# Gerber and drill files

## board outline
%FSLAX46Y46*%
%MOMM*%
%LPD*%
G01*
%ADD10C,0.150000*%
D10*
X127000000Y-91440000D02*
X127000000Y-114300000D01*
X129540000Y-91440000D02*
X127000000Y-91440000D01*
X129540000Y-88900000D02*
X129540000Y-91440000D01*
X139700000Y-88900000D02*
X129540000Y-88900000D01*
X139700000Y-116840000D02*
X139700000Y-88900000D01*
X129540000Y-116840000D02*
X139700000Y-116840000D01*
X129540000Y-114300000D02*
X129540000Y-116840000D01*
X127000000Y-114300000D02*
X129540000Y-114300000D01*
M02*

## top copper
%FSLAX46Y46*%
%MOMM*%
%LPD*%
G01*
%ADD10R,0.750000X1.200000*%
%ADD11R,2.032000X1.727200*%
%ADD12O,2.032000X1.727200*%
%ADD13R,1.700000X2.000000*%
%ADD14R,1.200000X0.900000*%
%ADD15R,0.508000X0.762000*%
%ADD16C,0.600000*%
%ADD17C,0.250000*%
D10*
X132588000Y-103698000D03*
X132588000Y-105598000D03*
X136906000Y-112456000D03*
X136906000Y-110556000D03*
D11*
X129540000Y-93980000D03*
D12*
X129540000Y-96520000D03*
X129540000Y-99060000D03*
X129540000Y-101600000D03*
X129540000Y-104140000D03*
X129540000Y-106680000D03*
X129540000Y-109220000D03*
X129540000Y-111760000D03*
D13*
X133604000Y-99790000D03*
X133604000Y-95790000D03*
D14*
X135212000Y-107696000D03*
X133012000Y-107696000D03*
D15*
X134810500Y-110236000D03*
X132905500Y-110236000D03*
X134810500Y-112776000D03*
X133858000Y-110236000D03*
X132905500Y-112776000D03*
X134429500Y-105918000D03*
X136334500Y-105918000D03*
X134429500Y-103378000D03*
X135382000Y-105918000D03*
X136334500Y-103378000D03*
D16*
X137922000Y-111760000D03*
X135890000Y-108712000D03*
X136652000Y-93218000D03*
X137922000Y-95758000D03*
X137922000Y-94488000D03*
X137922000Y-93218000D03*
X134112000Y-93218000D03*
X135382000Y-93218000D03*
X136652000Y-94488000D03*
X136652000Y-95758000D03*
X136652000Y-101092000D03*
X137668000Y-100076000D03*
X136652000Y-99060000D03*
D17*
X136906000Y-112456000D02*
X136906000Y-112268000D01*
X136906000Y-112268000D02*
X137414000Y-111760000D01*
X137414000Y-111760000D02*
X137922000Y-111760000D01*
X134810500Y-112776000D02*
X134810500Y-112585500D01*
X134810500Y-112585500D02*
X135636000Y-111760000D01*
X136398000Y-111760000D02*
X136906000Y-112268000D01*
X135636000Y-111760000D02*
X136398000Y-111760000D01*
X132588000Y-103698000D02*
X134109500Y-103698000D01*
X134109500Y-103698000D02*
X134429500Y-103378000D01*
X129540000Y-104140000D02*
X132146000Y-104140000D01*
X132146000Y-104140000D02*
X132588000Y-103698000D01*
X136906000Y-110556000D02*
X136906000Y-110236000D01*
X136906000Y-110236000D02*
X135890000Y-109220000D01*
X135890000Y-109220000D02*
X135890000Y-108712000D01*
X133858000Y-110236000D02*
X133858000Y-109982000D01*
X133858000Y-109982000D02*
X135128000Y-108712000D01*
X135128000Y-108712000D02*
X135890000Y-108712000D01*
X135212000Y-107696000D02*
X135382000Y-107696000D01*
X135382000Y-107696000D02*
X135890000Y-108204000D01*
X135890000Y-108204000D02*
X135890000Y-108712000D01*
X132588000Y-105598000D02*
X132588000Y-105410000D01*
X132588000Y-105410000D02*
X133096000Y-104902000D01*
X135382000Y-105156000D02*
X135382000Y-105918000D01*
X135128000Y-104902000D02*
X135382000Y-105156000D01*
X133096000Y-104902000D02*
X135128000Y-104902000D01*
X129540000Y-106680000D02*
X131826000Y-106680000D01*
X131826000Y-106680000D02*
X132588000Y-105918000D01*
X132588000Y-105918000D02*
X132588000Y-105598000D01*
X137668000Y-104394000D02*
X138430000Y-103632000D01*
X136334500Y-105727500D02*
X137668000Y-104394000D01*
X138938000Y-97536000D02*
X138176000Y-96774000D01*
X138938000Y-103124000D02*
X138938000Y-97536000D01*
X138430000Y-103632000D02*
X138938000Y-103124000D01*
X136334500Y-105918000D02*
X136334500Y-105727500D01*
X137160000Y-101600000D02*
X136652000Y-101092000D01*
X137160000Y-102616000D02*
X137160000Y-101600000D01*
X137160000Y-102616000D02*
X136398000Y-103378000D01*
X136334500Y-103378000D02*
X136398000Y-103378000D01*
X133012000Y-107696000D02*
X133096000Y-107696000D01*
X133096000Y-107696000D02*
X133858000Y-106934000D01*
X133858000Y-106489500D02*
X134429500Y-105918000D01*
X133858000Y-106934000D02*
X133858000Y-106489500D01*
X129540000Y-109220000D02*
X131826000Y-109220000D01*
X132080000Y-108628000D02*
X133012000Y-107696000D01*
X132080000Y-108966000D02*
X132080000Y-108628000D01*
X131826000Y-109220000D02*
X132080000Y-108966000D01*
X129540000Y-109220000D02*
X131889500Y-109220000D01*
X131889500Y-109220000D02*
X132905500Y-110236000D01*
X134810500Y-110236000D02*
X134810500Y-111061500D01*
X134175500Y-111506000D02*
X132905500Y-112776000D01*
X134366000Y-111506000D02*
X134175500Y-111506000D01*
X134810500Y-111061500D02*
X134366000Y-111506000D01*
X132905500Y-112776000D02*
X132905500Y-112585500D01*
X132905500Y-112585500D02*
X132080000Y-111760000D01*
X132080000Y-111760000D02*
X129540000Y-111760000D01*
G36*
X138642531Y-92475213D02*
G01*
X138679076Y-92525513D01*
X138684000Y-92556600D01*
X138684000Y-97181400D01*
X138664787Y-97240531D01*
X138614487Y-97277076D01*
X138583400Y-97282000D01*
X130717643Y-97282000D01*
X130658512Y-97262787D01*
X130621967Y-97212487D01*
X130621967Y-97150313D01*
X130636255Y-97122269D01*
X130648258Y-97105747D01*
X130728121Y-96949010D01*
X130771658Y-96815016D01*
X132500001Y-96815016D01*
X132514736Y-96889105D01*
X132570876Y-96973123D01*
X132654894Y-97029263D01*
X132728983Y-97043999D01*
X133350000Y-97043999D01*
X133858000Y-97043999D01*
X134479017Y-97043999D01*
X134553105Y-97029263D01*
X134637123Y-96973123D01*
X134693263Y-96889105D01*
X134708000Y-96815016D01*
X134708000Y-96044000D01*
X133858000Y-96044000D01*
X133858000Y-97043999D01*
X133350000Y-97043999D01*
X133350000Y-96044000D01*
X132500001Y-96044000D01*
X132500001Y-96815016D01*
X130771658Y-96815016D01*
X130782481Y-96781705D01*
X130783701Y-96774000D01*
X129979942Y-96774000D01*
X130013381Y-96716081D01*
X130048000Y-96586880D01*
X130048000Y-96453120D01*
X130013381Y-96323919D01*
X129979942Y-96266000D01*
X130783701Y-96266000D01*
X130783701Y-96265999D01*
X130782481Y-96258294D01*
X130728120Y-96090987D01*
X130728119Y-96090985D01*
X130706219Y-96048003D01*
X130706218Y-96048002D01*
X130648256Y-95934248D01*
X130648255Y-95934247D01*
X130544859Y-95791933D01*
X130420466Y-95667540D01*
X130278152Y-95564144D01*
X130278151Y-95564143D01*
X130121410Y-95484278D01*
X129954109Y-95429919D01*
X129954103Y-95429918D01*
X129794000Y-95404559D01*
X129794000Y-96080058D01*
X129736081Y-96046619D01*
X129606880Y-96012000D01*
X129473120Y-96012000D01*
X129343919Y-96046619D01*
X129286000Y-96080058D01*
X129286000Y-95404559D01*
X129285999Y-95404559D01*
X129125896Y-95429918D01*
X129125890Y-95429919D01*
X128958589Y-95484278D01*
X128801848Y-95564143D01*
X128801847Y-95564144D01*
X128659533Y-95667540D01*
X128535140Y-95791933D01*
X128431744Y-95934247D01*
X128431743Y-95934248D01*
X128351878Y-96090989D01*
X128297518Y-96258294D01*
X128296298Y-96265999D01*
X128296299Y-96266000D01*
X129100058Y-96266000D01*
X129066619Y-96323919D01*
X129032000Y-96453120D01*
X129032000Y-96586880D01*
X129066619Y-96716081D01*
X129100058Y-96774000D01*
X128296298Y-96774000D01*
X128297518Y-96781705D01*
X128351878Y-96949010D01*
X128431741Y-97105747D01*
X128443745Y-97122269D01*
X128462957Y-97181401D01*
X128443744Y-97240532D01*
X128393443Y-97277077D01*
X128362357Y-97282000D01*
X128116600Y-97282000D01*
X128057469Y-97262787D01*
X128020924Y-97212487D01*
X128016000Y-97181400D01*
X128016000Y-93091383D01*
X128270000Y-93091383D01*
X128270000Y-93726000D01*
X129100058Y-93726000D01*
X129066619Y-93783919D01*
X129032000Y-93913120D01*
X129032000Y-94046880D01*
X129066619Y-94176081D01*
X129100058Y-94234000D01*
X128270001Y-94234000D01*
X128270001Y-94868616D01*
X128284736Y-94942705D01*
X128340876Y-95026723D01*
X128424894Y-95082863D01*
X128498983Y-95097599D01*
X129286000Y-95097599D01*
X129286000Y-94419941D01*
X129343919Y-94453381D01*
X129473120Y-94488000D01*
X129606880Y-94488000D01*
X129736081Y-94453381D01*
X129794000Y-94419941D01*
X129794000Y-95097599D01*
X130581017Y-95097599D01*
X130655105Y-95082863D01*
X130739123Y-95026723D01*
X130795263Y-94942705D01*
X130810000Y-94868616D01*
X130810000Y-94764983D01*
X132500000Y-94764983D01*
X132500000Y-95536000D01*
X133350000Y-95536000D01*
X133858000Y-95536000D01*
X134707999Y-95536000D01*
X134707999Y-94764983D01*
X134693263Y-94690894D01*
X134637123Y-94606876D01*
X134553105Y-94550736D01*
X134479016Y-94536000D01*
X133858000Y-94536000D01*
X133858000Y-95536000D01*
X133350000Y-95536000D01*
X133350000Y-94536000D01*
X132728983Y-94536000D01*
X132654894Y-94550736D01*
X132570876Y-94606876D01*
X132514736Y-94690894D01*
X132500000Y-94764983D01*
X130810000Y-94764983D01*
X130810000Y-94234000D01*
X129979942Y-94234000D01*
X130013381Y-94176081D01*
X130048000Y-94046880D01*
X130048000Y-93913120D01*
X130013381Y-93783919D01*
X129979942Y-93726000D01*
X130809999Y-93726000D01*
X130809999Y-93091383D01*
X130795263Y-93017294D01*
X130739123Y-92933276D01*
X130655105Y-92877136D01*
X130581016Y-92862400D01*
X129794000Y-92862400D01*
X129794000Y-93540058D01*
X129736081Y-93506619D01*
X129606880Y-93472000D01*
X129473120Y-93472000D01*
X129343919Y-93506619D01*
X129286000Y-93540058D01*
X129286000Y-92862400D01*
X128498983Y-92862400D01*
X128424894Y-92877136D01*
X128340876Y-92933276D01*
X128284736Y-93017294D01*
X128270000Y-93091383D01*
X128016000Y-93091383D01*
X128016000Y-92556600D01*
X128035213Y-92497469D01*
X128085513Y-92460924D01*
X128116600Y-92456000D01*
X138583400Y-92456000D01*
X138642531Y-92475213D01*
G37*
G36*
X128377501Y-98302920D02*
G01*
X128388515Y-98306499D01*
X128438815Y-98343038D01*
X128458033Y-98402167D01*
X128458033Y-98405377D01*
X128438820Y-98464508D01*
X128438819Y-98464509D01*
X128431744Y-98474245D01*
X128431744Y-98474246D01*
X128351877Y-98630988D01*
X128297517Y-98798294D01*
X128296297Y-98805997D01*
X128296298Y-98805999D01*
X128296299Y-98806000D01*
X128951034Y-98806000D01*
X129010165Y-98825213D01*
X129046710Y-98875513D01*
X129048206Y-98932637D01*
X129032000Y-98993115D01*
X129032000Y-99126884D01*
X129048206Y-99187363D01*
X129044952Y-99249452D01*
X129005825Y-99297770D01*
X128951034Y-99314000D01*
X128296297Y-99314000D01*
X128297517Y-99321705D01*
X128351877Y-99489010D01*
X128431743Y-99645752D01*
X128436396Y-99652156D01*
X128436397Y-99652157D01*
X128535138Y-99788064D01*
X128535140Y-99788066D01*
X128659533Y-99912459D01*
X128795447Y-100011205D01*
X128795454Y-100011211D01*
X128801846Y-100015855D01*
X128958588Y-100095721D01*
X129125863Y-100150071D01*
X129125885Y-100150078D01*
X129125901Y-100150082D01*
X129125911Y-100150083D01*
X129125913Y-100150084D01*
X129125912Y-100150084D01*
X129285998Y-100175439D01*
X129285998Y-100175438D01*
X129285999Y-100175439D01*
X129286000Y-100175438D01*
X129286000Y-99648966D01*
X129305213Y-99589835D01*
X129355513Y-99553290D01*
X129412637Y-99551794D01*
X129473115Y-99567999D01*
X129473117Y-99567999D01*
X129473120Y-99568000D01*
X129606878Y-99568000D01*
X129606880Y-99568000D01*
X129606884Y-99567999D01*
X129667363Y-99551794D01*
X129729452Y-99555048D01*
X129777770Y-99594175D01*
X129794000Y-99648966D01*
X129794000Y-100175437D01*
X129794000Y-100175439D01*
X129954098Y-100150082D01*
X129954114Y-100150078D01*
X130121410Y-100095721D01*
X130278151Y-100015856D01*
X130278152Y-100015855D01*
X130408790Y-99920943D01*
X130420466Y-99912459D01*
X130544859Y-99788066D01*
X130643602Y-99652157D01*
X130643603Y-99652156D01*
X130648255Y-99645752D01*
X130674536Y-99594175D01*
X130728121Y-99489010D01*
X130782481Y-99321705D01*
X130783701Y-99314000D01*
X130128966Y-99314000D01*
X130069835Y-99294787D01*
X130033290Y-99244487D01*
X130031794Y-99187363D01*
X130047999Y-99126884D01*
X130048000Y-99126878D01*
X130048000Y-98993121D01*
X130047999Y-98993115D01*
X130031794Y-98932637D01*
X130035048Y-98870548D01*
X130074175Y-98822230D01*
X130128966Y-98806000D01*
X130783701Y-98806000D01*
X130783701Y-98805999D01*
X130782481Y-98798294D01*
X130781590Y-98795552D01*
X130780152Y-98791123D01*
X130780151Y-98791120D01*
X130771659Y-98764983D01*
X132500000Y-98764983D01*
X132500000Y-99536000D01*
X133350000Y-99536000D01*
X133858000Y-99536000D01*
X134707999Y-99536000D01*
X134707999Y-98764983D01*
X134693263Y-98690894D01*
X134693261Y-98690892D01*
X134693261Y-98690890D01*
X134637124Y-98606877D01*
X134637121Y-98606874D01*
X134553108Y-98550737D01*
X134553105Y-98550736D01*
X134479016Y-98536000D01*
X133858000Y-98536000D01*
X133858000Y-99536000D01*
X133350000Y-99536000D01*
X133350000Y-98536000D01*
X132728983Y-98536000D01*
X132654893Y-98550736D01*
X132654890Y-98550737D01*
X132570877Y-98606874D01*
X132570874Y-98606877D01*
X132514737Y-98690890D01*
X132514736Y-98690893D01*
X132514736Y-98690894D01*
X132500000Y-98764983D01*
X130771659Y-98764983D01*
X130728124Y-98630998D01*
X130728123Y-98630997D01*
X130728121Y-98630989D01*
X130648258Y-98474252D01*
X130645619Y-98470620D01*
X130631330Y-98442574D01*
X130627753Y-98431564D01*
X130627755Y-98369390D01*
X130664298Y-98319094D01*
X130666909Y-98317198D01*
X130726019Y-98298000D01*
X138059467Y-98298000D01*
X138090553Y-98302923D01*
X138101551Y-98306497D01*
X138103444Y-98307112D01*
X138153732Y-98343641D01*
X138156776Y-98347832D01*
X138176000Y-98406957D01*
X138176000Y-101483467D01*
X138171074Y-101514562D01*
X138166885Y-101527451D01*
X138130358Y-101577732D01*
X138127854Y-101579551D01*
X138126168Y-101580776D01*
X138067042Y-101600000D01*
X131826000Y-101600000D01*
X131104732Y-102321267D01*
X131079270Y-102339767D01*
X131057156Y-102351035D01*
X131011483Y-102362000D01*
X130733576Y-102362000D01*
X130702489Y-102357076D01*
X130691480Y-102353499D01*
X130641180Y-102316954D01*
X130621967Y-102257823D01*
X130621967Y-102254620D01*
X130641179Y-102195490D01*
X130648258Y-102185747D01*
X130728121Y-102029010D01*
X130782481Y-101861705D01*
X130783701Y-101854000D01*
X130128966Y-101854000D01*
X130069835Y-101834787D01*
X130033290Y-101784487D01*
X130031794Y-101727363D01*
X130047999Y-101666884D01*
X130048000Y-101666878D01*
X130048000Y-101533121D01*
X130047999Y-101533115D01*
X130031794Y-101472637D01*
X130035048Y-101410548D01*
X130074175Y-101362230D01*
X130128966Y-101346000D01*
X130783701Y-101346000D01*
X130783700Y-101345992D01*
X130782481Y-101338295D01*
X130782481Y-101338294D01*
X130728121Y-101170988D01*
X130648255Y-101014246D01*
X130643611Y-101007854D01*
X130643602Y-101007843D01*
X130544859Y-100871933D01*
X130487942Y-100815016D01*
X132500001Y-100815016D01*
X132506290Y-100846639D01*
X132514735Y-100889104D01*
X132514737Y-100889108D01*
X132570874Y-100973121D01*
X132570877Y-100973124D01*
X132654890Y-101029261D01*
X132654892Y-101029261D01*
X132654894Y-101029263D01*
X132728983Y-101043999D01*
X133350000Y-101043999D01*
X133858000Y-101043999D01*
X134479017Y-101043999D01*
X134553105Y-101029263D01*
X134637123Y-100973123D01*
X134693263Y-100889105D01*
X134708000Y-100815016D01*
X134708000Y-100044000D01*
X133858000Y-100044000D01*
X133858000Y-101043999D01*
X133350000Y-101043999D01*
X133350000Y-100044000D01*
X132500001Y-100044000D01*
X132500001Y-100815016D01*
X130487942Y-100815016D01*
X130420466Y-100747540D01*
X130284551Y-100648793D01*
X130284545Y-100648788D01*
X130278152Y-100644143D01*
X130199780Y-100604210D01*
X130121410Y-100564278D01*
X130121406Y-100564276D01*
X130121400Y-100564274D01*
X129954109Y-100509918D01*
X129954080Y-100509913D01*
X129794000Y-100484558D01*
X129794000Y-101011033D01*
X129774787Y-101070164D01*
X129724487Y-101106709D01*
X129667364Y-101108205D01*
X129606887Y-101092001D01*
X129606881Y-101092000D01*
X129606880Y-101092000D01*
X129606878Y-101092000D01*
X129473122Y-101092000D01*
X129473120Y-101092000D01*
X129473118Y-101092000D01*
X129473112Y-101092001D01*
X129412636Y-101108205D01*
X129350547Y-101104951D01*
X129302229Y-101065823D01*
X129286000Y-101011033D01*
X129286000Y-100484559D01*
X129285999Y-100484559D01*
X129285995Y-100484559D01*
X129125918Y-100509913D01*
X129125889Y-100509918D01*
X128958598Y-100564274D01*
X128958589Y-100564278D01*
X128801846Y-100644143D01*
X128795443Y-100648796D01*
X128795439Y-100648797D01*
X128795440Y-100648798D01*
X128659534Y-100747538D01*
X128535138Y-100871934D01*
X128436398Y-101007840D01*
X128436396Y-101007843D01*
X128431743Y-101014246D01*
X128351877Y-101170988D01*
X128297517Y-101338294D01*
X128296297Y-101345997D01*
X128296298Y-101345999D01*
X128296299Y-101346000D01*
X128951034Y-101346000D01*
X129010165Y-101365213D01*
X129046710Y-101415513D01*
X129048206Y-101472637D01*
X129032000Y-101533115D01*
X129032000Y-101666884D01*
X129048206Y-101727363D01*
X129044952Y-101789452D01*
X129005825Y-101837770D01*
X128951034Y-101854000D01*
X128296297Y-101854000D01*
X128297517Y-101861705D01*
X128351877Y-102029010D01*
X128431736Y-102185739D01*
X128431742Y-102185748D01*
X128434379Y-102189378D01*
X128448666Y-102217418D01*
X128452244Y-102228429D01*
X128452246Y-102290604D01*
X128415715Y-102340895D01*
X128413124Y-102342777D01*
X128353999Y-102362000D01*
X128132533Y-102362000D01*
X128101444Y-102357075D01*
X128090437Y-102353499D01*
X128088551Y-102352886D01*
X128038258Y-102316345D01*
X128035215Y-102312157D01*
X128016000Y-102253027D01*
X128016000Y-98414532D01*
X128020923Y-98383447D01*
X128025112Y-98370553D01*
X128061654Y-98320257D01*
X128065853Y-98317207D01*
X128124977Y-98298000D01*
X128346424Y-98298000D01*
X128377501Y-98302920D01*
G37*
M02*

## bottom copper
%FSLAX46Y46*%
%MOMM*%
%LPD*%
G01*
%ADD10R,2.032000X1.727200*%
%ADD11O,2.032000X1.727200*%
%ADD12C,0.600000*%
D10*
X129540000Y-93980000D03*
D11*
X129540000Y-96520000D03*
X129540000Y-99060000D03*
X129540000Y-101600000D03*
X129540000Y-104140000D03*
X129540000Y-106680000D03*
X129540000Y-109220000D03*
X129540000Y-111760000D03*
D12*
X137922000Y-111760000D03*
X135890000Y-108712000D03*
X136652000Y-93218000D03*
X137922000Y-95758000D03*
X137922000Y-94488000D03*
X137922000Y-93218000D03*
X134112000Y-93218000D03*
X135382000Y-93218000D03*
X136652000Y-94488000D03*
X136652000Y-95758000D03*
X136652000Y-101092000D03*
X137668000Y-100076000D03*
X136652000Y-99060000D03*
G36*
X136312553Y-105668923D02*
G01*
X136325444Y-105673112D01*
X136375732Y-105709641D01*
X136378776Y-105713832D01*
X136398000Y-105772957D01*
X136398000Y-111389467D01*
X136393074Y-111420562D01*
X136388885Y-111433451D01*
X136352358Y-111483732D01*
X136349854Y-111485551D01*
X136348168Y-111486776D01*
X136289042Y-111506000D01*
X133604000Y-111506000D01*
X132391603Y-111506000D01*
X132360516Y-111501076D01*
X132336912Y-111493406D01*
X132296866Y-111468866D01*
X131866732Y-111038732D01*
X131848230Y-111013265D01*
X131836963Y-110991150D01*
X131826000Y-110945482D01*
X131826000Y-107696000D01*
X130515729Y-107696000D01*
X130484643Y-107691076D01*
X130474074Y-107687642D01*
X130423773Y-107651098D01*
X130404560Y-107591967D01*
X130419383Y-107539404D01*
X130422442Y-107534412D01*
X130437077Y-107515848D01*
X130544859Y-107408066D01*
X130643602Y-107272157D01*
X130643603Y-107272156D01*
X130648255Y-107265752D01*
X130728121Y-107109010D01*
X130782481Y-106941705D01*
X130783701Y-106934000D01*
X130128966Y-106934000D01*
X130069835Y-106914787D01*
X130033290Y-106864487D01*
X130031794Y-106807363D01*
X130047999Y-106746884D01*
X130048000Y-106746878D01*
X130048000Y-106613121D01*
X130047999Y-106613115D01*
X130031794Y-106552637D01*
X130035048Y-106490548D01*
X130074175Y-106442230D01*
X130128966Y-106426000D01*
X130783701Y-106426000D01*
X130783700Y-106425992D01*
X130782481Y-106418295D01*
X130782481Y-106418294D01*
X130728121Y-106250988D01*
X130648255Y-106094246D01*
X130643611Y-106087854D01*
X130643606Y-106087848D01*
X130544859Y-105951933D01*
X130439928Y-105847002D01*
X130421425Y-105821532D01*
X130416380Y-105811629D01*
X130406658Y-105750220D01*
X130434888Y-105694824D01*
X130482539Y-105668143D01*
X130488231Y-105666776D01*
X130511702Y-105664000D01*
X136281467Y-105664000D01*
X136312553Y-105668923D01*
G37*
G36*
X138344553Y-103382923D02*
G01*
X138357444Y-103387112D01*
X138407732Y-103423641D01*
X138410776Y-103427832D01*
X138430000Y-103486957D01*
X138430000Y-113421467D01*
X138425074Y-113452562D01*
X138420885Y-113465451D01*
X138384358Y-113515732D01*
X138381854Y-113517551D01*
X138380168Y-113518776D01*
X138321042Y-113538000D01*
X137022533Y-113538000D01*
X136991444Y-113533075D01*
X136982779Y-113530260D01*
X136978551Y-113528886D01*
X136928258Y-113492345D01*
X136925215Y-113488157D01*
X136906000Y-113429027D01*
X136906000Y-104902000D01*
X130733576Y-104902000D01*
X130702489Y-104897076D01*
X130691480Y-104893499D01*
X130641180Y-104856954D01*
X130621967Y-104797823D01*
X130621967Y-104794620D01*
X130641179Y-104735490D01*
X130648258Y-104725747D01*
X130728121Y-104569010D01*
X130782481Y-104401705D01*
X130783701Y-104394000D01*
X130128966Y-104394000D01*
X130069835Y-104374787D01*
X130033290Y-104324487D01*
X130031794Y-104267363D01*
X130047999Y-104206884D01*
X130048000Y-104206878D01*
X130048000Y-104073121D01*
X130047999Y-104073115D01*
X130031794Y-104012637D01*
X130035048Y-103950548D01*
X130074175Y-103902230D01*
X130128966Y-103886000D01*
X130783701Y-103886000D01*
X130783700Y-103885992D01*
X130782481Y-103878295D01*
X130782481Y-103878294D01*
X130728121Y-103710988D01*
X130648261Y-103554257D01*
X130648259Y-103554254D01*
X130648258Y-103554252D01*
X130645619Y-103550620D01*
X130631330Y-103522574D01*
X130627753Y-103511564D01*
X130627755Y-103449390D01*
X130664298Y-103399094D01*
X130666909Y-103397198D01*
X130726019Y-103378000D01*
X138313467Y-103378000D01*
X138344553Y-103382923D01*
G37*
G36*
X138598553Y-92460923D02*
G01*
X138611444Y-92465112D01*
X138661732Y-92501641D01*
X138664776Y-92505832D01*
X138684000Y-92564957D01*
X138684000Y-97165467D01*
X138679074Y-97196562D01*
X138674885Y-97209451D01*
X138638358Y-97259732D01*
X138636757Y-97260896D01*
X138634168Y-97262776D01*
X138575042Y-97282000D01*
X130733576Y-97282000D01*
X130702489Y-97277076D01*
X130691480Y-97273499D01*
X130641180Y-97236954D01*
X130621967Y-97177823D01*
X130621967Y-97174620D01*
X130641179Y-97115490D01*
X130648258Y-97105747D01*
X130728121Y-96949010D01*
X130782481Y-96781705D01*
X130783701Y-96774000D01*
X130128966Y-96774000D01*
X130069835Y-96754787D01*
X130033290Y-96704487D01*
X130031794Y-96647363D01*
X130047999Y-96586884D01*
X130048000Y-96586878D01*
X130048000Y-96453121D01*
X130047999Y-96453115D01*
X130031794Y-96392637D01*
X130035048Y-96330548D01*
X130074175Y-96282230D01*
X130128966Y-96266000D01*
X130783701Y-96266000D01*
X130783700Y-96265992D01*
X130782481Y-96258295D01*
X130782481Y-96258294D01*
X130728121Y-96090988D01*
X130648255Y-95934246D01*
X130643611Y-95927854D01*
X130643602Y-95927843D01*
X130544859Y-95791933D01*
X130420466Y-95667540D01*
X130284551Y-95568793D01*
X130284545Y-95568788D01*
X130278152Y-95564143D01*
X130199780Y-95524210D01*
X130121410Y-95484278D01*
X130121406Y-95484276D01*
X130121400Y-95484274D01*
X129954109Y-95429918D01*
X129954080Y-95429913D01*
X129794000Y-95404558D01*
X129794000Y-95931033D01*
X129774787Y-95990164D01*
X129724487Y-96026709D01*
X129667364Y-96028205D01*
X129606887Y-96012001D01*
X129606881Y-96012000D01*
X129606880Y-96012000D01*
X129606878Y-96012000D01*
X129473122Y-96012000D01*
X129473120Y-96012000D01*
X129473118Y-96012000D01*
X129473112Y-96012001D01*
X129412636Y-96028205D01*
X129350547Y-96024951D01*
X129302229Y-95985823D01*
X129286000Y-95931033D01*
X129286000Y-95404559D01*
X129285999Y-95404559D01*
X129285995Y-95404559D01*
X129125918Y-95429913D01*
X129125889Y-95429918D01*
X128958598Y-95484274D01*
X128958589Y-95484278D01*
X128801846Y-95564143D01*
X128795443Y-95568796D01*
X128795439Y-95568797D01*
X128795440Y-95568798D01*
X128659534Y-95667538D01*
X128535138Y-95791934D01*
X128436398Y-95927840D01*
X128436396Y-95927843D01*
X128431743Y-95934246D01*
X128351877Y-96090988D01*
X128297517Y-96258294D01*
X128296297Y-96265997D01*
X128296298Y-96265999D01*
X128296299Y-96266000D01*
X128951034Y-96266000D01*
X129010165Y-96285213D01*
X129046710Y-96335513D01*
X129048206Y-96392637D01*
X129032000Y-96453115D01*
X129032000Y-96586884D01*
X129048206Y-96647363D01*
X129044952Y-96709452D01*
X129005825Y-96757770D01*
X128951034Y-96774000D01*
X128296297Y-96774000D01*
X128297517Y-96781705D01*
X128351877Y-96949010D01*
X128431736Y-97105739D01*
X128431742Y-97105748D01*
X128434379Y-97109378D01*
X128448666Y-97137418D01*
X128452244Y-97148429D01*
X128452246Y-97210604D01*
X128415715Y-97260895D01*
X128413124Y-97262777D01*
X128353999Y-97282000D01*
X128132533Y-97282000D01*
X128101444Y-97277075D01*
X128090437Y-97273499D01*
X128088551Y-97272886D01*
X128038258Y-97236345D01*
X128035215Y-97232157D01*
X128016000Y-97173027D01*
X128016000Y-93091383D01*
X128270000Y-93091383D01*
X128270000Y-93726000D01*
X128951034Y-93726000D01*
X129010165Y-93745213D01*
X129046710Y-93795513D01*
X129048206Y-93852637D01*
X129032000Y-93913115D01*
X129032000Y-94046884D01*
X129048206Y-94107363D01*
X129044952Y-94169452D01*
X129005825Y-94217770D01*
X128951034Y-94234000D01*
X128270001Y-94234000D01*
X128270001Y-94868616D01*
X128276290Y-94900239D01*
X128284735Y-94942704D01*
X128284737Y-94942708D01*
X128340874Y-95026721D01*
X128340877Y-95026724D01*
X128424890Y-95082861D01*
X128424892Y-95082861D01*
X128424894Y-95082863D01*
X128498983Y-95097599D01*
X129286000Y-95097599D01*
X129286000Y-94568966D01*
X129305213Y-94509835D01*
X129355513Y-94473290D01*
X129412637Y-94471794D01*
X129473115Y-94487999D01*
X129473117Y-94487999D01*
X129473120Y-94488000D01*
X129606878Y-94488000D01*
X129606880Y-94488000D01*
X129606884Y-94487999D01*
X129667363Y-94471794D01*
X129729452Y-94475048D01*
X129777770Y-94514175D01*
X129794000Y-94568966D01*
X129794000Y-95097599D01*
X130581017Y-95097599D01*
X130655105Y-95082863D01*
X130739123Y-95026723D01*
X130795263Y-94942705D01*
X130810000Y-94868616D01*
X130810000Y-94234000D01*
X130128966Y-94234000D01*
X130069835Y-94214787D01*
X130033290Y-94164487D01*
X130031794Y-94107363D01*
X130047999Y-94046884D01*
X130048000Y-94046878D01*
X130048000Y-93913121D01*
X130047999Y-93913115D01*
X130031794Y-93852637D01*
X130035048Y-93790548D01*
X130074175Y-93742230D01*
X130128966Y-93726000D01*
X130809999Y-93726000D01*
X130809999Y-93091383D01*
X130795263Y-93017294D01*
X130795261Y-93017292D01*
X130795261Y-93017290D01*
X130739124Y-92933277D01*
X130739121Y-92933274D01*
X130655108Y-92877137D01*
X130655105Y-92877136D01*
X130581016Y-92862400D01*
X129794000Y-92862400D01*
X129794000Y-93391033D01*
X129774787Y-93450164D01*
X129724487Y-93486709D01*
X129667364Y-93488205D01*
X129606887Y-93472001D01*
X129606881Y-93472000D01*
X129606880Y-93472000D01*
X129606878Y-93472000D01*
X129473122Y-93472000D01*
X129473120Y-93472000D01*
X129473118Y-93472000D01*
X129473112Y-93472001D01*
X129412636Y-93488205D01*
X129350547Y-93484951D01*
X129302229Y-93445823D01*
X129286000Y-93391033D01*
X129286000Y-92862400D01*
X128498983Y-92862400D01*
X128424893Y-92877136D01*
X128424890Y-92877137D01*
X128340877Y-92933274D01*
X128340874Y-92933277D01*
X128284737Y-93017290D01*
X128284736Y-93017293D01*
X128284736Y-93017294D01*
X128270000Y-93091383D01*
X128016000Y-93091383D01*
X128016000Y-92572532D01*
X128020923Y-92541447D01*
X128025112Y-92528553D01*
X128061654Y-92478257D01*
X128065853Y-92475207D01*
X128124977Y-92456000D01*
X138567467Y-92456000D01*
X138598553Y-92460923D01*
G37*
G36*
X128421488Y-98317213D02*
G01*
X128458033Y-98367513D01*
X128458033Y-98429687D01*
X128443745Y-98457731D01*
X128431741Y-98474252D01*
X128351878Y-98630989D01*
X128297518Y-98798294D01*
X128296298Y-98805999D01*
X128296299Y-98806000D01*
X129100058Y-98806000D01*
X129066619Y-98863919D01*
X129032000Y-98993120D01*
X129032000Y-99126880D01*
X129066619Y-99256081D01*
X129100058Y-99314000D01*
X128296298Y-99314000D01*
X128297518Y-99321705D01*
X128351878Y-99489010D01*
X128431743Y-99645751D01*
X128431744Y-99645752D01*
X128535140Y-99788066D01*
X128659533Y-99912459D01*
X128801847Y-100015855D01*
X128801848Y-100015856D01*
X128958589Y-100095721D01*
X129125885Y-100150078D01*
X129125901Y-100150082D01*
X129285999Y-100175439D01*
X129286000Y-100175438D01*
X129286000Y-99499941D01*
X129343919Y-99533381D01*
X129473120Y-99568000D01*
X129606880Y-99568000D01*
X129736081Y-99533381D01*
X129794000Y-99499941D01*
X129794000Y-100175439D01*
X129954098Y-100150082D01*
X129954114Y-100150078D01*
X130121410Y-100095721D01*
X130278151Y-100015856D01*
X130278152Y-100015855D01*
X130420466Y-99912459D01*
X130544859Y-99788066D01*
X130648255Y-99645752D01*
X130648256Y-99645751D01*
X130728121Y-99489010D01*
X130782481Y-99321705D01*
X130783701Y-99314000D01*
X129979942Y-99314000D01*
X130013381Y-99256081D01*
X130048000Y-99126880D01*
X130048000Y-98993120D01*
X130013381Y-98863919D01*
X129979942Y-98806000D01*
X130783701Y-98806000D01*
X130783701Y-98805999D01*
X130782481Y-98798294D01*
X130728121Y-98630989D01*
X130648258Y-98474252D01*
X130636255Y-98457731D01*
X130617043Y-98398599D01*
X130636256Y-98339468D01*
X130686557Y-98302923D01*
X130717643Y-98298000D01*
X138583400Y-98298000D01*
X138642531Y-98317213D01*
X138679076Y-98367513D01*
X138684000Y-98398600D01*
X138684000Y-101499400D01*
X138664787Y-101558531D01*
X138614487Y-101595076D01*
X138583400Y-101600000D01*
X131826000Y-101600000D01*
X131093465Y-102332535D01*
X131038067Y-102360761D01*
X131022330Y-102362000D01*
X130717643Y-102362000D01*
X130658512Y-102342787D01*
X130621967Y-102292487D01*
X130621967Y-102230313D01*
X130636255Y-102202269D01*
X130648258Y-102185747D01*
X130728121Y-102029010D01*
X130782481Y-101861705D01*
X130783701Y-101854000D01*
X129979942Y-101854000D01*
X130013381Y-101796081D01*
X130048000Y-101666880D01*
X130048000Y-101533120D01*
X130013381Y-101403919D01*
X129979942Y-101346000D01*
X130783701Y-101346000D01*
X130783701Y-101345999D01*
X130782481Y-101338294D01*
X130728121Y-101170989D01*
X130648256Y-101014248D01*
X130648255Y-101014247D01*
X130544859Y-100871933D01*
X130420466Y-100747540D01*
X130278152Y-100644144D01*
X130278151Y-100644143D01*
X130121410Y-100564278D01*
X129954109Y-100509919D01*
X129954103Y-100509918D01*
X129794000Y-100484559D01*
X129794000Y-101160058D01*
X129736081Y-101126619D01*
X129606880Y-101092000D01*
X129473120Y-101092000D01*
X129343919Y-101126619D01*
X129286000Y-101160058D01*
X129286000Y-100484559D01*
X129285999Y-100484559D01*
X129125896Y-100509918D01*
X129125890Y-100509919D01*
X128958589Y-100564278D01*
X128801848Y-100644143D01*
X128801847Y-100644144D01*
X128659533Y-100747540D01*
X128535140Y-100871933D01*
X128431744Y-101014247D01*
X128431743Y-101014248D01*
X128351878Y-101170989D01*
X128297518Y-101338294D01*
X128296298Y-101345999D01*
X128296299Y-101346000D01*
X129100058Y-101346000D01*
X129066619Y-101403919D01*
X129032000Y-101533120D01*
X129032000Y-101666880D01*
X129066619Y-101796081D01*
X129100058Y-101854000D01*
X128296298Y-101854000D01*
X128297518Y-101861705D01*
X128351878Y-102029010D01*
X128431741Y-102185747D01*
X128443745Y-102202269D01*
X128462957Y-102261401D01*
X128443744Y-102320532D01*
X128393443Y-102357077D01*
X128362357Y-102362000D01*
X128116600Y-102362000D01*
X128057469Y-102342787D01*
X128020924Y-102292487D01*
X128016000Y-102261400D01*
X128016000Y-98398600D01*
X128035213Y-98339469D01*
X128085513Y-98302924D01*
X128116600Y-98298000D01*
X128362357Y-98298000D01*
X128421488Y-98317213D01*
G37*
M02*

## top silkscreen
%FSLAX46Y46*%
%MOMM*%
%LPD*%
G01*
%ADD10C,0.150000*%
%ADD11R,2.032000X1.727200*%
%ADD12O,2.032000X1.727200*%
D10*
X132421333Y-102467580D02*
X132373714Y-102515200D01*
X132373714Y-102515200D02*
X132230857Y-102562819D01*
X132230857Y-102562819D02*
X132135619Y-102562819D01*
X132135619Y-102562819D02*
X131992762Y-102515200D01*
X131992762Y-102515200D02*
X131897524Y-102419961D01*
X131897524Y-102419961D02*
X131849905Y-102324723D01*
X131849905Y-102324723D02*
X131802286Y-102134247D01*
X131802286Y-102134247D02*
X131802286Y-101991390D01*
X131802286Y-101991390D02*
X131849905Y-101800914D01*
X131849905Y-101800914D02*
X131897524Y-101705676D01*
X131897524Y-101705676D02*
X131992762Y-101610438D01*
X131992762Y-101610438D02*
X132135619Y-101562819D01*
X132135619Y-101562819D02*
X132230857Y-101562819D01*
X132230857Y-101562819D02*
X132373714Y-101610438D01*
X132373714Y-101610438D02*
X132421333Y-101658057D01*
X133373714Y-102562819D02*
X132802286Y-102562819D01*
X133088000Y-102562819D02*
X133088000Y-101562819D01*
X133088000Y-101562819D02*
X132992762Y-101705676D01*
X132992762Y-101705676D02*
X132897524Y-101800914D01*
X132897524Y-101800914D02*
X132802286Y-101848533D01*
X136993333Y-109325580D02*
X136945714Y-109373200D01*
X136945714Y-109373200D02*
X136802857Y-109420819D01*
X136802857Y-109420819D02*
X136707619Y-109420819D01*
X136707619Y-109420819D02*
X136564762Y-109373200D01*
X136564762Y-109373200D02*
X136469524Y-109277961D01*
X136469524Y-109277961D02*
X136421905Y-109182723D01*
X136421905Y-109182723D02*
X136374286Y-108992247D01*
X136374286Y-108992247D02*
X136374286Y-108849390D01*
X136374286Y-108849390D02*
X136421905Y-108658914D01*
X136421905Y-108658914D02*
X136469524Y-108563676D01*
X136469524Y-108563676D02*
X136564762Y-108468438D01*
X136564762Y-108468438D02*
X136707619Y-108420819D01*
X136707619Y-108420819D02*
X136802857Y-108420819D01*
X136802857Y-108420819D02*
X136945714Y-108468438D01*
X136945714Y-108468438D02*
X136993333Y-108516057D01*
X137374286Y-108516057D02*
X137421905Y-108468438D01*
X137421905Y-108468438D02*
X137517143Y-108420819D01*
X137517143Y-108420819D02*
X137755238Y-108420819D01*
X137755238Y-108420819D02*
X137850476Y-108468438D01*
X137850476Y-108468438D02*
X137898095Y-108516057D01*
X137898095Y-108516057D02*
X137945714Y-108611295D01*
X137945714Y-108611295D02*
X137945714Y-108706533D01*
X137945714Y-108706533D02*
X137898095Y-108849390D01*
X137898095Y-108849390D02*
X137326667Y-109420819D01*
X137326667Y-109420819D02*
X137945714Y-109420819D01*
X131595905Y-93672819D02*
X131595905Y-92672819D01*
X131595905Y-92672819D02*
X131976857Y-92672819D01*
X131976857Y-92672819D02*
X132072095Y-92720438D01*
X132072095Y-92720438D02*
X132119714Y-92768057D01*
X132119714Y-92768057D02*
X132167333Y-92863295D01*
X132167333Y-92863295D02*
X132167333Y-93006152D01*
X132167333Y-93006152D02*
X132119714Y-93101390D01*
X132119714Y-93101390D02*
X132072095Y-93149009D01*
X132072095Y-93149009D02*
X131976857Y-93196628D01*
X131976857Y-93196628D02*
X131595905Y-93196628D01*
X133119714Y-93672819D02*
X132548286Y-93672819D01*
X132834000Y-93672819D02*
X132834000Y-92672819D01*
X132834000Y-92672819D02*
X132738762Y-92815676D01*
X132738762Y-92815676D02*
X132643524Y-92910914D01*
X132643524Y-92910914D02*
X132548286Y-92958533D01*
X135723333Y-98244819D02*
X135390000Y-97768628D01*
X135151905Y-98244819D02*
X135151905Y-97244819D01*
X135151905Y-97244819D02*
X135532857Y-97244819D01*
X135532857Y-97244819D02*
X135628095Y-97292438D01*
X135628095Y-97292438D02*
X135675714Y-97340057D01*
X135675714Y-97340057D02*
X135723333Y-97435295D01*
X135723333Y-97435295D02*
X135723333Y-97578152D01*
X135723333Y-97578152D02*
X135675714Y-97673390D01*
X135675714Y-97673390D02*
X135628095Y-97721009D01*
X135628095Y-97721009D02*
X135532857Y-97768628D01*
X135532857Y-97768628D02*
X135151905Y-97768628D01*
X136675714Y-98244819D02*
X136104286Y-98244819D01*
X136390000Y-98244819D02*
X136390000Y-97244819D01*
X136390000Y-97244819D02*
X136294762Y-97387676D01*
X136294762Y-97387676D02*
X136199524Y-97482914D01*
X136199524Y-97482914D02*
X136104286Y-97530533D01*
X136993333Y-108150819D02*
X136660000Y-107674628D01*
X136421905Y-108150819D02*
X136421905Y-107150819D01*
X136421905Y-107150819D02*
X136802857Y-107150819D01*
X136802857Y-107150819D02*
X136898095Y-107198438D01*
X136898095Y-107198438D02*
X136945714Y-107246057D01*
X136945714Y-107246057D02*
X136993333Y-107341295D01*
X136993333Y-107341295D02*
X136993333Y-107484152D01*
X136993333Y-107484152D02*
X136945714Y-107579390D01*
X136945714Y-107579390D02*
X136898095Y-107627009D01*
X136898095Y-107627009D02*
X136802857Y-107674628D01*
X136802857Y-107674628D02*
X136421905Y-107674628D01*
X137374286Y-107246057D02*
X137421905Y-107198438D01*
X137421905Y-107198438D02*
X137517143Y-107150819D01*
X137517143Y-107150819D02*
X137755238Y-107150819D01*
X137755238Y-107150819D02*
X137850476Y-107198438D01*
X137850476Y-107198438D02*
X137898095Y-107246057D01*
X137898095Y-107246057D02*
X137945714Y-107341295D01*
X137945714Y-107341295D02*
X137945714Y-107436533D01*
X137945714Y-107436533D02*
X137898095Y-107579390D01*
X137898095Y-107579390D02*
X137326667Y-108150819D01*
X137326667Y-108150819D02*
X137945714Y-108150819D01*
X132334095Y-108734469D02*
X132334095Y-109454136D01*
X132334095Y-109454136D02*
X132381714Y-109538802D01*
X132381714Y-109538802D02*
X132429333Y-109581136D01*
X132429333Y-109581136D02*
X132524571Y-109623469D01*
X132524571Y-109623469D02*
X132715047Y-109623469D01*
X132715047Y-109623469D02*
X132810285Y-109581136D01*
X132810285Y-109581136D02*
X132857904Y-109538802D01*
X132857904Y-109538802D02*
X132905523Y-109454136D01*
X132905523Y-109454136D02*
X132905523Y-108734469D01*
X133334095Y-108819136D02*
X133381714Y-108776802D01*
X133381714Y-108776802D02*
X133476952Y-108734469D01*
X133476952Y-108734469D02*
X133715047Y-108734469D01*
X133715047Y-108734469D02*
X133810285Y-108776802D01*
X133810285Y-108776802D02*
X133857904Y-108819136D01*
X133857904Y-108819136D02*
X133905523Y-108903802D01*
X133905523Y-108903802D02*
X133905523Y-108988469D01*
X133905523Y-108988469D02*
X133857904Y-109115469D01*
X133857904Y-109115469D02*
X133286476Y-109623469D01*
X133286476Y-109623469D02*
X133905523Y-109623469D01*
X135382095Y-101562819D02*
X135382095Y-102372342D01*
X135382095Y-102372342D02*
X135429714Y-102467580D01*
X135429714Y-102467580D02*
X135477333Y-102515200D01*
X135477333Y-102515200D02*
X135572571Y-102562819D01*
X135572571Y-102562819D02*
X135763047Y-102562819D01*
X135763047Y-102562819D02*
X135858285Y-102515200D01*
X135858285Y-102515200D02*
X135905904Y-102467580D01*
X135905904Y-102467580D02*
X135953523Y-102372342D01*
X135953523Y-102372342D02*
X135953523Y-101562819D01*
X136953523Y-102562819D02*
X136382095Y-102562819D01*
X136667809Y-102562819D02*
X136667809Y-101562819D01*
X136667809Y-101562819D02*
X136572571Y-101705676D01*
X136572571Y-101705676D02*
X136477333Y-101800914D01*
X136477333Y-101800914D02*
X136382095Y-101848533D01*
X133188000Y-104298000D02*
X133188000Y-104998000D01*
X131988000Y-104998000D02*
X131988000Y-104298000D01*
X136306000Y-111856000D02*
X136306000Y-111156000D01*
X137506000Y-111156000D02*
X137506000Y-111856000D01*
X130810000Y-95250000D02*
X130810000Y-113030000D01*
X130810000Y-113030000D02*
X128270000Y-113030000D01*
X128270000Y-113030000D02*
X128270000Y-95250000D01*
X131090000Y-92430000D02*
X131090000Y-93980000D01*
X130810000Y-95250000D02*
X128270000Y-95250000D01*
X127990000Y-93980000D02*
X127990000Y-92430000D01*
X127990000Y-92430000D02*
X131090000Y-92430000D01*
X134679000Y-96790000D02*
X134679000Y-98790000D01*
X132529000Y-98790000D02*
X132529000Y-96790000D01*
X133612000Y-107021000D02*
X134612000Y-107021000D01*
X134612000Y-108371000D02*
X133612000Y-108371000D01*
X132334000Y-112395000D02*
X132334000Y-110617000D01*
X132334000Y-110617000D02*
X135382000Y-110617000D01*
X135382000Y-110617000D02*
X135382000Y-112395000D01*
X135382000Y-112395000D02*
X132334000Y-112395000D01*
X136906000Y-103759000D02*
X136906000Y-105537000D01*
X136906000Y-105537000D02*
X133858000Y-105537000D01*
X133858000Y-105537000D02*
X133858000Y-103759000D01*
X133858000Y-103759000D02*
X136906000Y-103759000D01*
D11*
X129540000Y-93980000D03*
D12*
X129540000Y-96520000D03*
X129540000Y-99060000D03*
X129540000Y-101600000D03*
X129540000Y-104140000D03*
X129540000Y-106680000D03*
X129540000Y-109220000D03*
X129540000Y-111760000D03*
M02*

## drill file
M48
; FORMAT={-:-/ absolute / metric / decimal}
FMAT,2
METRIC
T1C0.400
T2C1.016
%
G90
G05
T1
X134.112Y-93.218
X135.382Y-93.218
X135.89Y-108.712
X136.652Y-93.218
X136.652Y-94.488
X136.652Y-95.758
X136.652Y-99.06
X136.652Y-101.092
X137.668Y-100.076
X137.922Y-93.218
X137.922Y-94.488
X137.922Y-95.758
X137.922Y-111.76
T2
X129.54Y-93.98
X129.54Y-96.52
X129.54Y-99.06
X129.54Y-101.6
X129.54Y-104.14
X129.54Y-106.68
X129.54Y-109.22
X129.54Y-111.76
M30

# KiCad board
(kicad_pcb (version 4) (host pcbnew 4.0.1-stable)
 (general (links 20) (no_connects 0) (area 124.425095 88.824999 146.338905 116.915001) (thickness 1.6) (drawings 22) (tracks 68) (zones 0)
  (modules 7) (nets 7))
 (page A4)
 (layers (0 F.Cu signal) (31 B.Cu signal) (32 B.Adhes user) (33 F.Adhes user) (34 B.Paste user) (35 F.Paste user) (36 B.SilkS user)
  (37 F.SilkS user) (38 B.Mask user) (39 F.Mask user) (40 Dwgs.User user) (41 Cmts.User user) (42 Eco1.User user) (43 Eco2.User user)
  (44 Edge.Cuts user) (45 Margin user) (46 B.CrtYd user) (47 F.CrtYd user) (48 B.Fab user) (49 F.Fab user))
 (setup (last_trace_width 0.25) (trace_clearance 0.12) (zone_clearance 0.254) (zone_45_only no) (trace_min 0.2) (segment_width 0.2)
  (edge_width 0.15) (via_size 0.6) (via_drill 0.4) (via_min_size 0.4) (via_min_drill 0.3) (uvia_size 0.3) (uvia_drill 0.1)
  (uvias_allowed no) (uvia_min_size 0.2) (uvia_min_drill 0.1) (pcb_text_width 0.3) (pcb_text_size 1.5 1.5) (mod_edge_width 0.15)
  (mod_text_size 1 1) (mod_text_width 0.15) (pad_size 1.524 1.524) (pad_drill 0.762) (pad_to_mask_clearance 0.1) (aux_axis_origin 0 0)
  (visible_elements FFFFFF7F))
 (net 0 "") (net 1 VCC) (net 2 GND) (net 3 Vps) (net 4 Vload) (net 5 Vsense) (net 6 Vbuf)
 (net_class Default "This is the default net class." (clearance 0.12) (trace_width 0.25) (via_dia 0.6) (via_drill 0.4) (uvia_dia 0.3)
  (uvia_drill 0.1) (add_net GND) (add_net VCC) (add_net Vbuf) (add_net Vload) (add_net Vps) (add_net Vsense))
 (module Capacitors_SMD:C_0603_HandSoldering (layer F.Cu) (at 132.588 104.648 270)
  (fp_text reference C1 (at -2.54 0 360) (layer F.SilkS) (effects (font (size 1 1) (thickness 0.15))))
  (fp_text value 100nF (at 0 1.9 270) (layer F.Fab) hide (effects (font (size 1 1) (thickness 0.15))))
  (fp_line (start -0.35 -0.6) (end 0.35 -0.6) (layer F.SilkS) (width 0.15))
  (fp_line (start 0.35 0.6) (end -0.35 0.6) (layer F.SilkS) (width 0.15))
  (pad 1 smd rect (at -0.95 0 270) (size 1.2 0.75) (layers F.Cu F.Paste F.Mask) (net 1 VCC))
  (pad 2 smd rect (at 0.95 0 270) (size 1.2 0.75) (layers F.Cu F.Paste F.Mask) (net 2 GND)))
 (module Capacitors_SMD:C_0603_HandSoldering (layer F.Cu) (at 136.906 111.506 90)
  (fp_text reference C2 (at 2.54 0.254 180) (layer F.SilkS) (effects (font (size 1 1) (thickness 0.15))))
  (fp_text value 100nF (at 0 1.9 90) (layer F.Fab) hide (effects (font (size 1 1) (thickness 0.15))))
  (fp_line (start -0.35 -0.6) (end 0.35 -0.6) (layer F.SilkS) (width 0.15))
  (fp_line (start 0.35 0.6) (end -0.35 0.6) (layer F.SilkS) (width 0.15))
  (pad 1 smd rect (at -0.95 0 90) (size 1.2 0.75) (layers F.Cu F.Paste F.Mask) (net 1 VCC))
  (pad 2 smd rect (at 0.95 0 90) (size 1.2 0.75) (layers F.Cu F.Paste F.Mask) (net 2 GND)))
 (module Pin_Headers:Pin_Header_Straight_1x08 (layer F.Cu) (at 129.54 93.98)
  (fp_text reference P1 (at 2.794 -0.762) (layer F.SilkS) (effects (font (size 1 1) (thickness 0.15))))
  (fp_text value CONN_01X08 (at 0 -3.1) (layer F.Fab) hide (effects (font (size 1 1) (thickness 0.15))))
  (fp_line (start 1.27 1.27) (end 1.27 19.05) (layer F.SilkS) (width 0.15))
  (fp_line (start 1.27 19.05) (end -1.27 19.05) (layer F.SilkS) (width 0.15))
  (fp_line (start -1.27 19.05) (end -1.27 1.27) (layer F.SilkS) (width 0.15))
  (fp_line (start 1.55 -1.55) (end 1.55 0) (layer F.SilkS) (width 0.15))
  (fp_line (start 1.27 1.27) (end -1.27 1.27) (layer F.SilkS) (width 0.15))
  (fp_line (start -1.55 0) (end -1.55 -1.55) (layer F.SilkS) (width 0.15))
  (fp_line (start -1.55 -1.55) (end 1.55 -1.55) (layer F.SilkS) (width 0.15))
  (pad 1 thru_hole rect (at 0 0) (size 2.032 1.7272) (drill 1.016) (layers *.Cu *.Mask F.SilkS) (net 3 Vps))
  (pad 2 thru_hole oval (at 0 2.54) (size 2.032 1.7272) (drill 1.016) (layers *.Cu *.Mask F.SilkS) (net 3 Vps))
  (pad 3 thru_hole oval (at 0 5.08) (size 2.032 1.7272) (drill 1.016) (layers *.Cu *.Mask F.SilkS) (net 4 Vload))
  (pad 4 thru_hole oval (at 0 7.62) (size 2.032 1.7272) (drill 1.016) (layers *.Cu *.Mask F.SilkS) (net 4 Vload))
  (pad 5 thru_hole oval (at 0 10.16) (size 2.032 1.7272) (drill 1.016) (layers *.Cu *.Mask F.SilkS) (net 1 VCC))
  (pad 6 thru_hole oval (at 0 12.7) (size 2.032 1.7272) (drill 1.016) (layers *.Cu *.Mask F.SilkS) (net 2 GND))
  (pad 7 thru_hole oval (at 0 15.24) (size 2.032 1.7272) (drill 1.016) (layers *.Cu *.Mask F.SilkS) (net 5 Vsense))
  (pad 8 thru_hole oval (at 0 17.78) (size 2.032 1.7272) (drill 1.016) (layers *.Cu *.Mask F.SilkS) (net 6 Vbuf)))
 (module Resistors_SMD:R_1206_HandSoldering (layer F.Cu) (at 133.604 97.79 90)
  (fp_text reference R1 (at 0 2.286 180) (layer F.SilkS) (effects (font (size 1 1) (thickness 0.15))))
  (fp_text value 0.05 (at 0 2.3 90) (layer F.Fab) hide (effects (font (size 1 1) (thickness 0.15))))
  (fp_line (start 1 1.075) (end -1 1.075) (layer F.SilkS) (width 0.15))
  (fp_line (start -1 -1.075) (end 1 -1.075) (layer F.SilkS) (width 0.15))
  (pad 1 smd rect (at -2 0 90) (size 2 1.7) (layers F.Cu F.Paste F.Mask) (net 4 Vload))
  (pad 2 smd rect (at 2 0 90) (size 2 1.7) (layers F.Cu F.Paste F.Mask) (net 3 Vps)))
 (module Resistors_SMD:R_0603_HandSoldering (layer F.Cu) (at 134.112 107.696 180)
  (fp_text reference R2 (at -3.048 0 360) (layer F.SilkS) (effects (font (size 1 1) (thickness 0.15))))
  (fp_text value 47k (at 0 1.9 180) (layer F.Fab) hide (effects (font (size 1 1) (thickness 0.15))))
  (fp_line (start 0.5 0.675) (end -0.5 0.675) (layer F.SilkS) (width 0.15))
  (fp_line (start -0.5 -0.675) (end 0.5 -0.675) (layer F.SilkS) (width 0.15))
  (pad 1 smd rect (at -1.1 0 180) (size 1.2 0.9) (layers F.Cu F.Paste F.Mask) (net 2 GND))
  (pad 2 smd rect (at 1.1 0 180) (size 1.2 0.9) (layers F.Cu F.Paste F.Mask) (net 5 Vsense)))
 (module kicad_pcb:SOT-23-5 (layer F.Cu) (at 133.858 111.506 180)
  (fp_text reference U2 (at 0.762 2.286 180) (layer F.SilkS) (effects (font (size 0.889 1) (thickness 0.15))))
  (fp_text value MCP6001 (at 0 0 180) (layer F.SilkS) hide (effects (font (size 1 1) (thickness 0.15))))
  (fp_line (start 1.524 -0.889) (end 1.524 0.889) (layer F.SilkS) (width 0.15))
  (fp_line (start 1.524 0.889) (end -1.524 0.889) (layer F.SilkS) (width 0.15))
  (fp_line (start -1.524 0.889) (end -1.524 -0.889) (layer F.SilkS) (width 0.15))
  (fp_line (start -1.524 -0.889) (end 1.524 -0.889) (layer F.SilkS) (width 0.15))
  (pad 1 smd rect (at -0.9525 1.27 180) (size 0.508 0.762) (layers F.Cu F.Paste F.Mask) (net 6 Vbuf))
  (pad 3 smd rect (at 0.9525 1.27 180) (size 0.508 0.762) (layers F.Cu F.Paste F.Mask) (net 5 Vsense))
  (pad 5 smd rect (at -0.9525 -1.27 180) (size 0.508 0.762) (layers F.Cu F.Paste F.Mask) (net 1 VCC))
  (pad 2 smd rect (at 0 1.27 180) (size 0.508 0.762) (layers F.Cu F.Paste F.Mask) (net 2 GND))
  (pad 4 smd rect (at 0.9525 -1.27 180) (size 0.508 0.762) (layers F.Cu F.Paste F.Mask) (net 6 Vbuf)))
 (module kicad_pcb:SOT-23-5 (layer F.Cu) (at 135.382 104.648)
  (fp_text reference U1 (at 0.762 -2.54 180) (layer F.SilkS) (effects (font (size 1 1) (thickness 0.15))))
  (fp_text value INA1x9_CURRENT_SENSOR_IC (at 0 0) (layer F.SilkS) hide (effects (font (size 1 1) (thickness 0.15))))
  (fp_line (start 1.524 -0.889) (end 1.524 0.889) (layer F.SilkS) (width 0.15))
  (fp_line (start 1.524 0.889) (end -1.524 0.889) (layer F.SilkS) (width 0.15))
  (fp_line (start -1.524 0.889) (end -1.524 -0.889) (layer F.SilkS) (width 0.15))
  (fp_line (start -1.524 -0.889) (end 1.524 -0.889) (layer F.SilkS) (width 0.15))
  (pad 1 smd rect (at -0.9525 1.27) (size 0.508 0.762) (layers F.Cu F.Paste F.Mask) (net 5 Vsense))
  (pad 3 smd rect (at 0.9525 1.27) (size 0.508 0.762) (layers F.Cu F.Paste F.Mask) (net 3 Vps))
  (pad 5 smd rect (at -0.9525 -1.27) (size 0.508 0.762) (layers F.Cu F.Paste F.Mask) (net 1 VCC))
  (pad 2 smd rect (at 0 1.27) (size 0.508 0.762) (layers F.Cu F.Paste F.Mask) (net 2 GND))
  (pad 4 smd rect (at 0.9525 -1.27) (size 0.508 0.762) (layers F.Cu F.Paste F.Mask) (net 4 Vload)))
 (gr_line (start 127 91.44) (end 127 114.3) (angle 90) (layer Edge.Cuts) (width 0.15))
 (gr_line (start 129.54 91.44) (end 127 91.44) (angle 90) (layer Edge.Cuts) (width 0.15))
 (gr_line (start 129.54 88.9) (end 129.54 91.44) (angle 90) (layer Edge.Cuts) (width 0.15))
 (gr_line (start 139.7 88.9) (end 129.54 88.9) (angle 90) (layer Edge.Cuts) (width 0.15))
 (gr_line (start 139.7 116.84) (end 139.7 88.9) (angle 90) (layer Edge.Cuts) (width 0.15))
 (gr_line (start 129.54 116.84) (end 139.7 116.84) (angle 90) (layer Edge.Cuts) (width 0.15))
 (gr_line (start 129.54 114.3) (end 129.54 116.84) (angle 90) (layer Edge.Cuts) (width 0.15))
 (gr_line (start 127 114.3) (end 129.54 114.3) (angle 90) (layer Edge.Cuts) (width 0.15))
 (segment (start 136.906 112.456) (end 136.906 112.268) (width 0.25) (layer F.Cu) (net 1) (status C00000))
 (segment (start 136.906 112.268) (end 137.414 111.76) (width 0.25) (layer F.Cu) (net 1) (status 400000))
 (via (at 137.922 111.76) (size 0.6) (drill 0.4) (layers F.Cu B.Cu) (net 1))
 (segment (start 137.414 111.76) (end 137.922 111.76) (width 0.25) (layer F.Cu) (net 1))
 (segment (start 134.8105 112.776) (end 134.8105 112.5855) (width 0.25) (layer F.Cu) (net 1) (status C00000))
 (segment (start 134.8105 112.5855) (end 135.636 111.76) (width 0.25) (layer F.Cu) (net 1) (status 400000))
 (segment (start 136.398 111.76) (end 136.906 112.268) (width 0.25) (layer F.Cu) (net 1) (status 800000))
 (segment (start 135.636 111.76) (end 136.398 111.76) (width 0.25) (layer F.Cu) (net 1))
 (segment (start 132.588 103.698) (end 134.1095 103.698) (width 0.25) (layer F.Cu) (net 1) (status 400000))
 (segment (start 134.1095 103.698) (end 134.4295 103.378) (width 0.25) (layer F.Cu) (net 1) (status 800000))
 (segment (start 129.54 104.14) (end 132.146 104.14) (width 0.25) (layer F.Cu) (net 1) (status 400000))
 (segment (start 132.146 104.14) (end 132.588 103.698) (width 0.25) (layer F.Cu) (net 1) (status 800000))
 (segment (start 136.906 110.556) (end 136.906 110.236) (width 0.25) (layer F.Cu) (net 2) (status C00000))
 (segment (start 136.906 110.236) (end 135.89 109.22) (width 0.25) (layer F.Cu) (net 2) (status 400000))
 (segment (start 135.89 109.22) (end 135.89 108.712) (width 0.25) (layer F.Cu) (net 2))
 (segment (start 133.858 110.236) (end 133.858 109.982) (width 0.25) (layer F.Cu) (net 2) (status C00000))
 (segment (start 133.858 109.982) (end 135.128 108.712) (width 0.25) (layer F.Cu) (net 2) (status 400000))
 (segment (start 135.128 108.712) (end 135.89 108.712) (width 0.25) (layer F.Cu) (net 2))
 (segment (start 135.212 107.696) (end 135.382 107.696) (width 0.25) (layer F.Cu) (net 2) (status C00000))
 (segment (start 135.382 107.696) (end 135.89 108.204) (width 0.25) (layer F.Cu) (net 2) (status 400000))
 (segment (start 135.89 108.204) (end 135.89 108.712) (width 0.25) (layer F.Cu) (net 2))
 (via (at 135.89 108.712) (size 0.6) (drill 0.4) (layers F.Cu B.Cu) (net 2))
 (segment (start 132.588 105.598) (end 132.588 105.41) (width 0.25) (layer F.Cu) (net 2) (status C00000))
 (segment (start 132.588 105.41) (end 133.096 104.902) (width 0.25) (layer F.Cu) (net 2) (status 400000))
 (segment (start 135.382 105.156) (end 135.382 105.918) (width 0.25) (layer F.Cu) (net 2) (status 800000))
 (segment (start 135.128 104.902) (end 135.382 105.156) (width 0.25) (layer F.Cu) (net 2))
 (segment (start 133.096 104.902) (end 135.128 104.902) (width 0.25) (layer F.Cu) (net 2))
 (segment (start 129.54 106.68) (end 131.826 106.68) (width 0.25) (layer F.Cu) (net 2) (status 400000))
 (segment (start 131.826 106.68) (end 132.588 105.918) (width 0.25) (layer F.Cu) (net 2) (status 800000))
 (segment (start 132.588 105.918) (end 132.588 105.598) (width 0.25) (layer F.Cu) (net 2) (status C00000))
 (via (at 136.652 93.218) (size 0.6) (drill 0.4) (layers F.Cu B.Cu) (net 3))
 (via (at 137.922 95.758) (size 0.6) (drill 0.4) (layers F.Cu B.Cu) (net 3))
 (via (at 137.922 94.488) (size 0.6) (drill 0.4) (layers F.Cu B.Cu) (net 3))
 (via (at 137.922 93.218) (size 0.6) (drill 0.4) (layers F.Cu B.Cu) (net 3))
 (segment (start 137.668 104.394) (end 138.43 103.632) (width 0.25) (layer F.Cu) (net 3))
 (segment (start 136.3345 105.7275) (end 137.668 104.394) (width 0.25) (layer F.Cu) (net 3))
 (segment (start 138.938 97.536) (end 138.176 96.774) (width 0.25) (layer F.Cu) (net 3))
 (segment (start 138.938 103.124) (end 138.938 97.536) (width 0.25) (layer F.Cu) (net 3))
 (segment (start 138.43 103.632) (end 138.938 103.124) (width 0.25) (layer F.Cu) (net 3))
 (via (at 134.112 93.218) (size 0.6) (drill 0.4) (layers F.Cu B.Cu) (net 3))
 (via (at 135.382 93.218) (size 0.6) (drill 0.4) (layers F.Cu B.Cu) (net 3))
 (via (at 136.652 94.488) (size 0.6) (drill 0.4) (layers F.Cu B.Cu) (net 3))
 (via (at 136.652 95.758) (size 0.6) (drill 0.4) (layers F.Cu B.Cu) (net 3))
 (segment (start 136.3345 105.918) (end 136.3345 105.7275) (width 0.25) (layer F.Cu) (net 3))
 (segment (start 137.16 101.6) (end 136.652 101.092) (width 0.25) (layer F.Cu) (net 4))
 (segment (start 137.16 102.616) (end 137.16 101.6) (width 0.25) (layer F.Cu) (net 4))
 (segment (start 137.16 102.616) (end 136.398 103.378) (width 0.25) (layer F.Cu) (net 4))
 (via (at 136.652 101.092) (size 0.6) (drill 0.4) (layers F.Cu B.Cu) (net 4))
 (via (at 137.668 100.076) (size 0.6) (drill 0.4) (layers F.Cu B.Cu) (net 4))
 (via (at 136.652 99.06) (size 0.6) (drill 0.4) (layers F.Cu B.Cu) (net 4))
 (segment (start 136.3345 103.378) (end 136.398 103.378) (width 0.25) (layer F.Cu) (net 4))
 (segment (start 133.012 107.696) (end 133.096 107.696) (width 0.25) (layer F.Cu) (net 5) (status C00000))
 (segment (start 133.096 107.696) (end 133.858 106.934) (width 0.25) (layer F.Cu) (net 5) (status 400000))
 (segment (start 133.858 106.4895) (end 134.4295 105.918) (width 0.25) (layer F.Cu) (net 5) (status 800000))
 (segment (start 133.858 106.934) (end 133.858 106.4895) (width 0.25) (layer F.Cu) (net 5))
 (segment (start 129.54 109.22) (end 131.826 109.22) (width 0.25) (layer F.Cu) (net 5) (status 400000))
 (segment (start 132.08 108.628) (end 133.012 107.696) (width 0.25) (layer F.Cu) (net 5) (status 800000))
 (segment (start 132.08 108.966) (end 132.08 108.628) (width 0.25) (layer F.Cu) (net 5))
 (segment (start 131.826 109.22) (end 132.08 108.966) (width 0.25) (layer F.Cu) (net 5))
 (segment (start 129.54 109.22) (end 131.8895 109.22) (width 0.25) (layer F.Cu) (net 5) (status 400000))
 (segment (start 131.8895 109.22) (end 132.9055 110.236) (width 0.25) (layer F.Cu) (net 5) (status 800000))
 (segment (start 134.8105 110.236) (end 134.8105 111.0615) (width 0.25) (layer F.Cu) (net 6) (status 400000))
 (segment (start 134.1755 111.506) (end 132.9055 112.776) (width 0.25) (layer F.Cu) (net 6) (status 800000))
 (segment (start 134.366 111.506) (end 134.1755 111.506) (width 0.25) (layer F.Cu) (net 6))
 (segment (start 134.8105 111.0615) (end 134.366 111.506) (width 0.25) (layer F.Cu) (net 6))
 (segment (start 132.9055 112.776) (end 132.9055 112.5855) (width 0.25) (layer F.Cu) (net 6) (status C00000))
 (segment (start 132.9055 112.5855) (end 132.08 111.76) (width 0.25) (layer F.Cu) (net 6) (status 400000))
 (segment (start 132.08 111.76) (end 129.54 111.76) (width 0.25) (layer F.Cu) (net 6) (status 800000))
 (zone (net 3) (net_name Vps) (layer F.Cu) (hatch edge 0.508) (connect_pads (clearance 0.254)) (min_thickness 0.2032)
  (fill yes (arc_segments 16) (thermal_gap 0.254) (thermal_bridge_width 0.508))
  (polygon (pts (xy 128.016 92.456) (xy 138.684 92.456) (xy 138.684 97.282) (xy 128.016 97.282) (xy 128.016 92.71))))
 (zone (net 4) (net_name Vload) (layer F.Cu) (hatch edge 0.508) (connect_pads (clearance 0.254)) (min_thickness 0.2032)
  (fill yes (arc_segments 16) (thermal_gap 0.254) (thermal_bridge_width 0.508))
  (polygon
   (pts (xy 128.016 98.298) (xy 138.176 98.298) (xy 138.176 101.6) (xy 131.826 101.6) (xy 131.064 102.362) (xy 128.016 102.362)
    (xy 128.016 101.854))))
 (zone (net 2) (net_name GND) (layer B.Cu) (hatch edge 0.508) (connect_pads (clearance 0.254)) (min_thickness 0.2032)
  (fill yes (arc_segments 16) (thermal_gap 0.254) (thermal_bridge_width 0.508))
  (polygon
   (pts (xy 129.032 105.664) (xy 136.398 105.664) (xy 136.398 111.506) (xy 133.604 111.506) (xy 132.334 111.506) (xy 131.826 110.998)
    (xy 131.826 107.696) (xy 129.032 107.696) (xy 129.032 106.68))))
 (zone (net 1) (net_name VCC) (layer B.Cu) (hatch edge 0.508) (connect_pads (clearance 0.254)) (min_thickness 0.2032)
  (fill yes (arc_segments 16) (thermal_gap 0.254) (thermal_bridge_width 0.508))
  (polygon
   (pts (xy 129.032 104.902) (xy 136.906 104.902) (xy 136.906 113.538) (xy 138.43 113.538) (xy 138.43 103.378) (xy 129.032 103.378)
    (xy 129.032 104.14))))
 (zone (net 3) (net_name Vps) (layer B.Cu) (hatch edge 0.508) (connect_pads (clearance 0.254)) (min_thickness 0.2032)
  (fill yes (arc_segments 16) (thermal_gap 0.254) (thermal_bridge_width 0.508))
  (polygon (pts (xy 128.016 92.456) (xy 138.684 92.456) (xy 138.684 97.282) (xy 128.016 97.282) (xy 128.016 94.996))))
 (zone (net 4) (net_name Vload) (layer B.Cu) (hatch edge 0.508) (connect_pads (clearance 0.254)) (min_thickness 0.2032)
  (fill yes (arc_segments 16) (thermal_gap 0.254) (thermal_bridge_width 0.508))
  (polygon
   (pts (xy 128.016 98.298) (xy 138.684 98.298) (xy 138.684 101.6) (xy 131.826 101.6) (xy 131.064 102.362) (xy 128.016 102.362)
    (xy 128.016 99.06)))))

